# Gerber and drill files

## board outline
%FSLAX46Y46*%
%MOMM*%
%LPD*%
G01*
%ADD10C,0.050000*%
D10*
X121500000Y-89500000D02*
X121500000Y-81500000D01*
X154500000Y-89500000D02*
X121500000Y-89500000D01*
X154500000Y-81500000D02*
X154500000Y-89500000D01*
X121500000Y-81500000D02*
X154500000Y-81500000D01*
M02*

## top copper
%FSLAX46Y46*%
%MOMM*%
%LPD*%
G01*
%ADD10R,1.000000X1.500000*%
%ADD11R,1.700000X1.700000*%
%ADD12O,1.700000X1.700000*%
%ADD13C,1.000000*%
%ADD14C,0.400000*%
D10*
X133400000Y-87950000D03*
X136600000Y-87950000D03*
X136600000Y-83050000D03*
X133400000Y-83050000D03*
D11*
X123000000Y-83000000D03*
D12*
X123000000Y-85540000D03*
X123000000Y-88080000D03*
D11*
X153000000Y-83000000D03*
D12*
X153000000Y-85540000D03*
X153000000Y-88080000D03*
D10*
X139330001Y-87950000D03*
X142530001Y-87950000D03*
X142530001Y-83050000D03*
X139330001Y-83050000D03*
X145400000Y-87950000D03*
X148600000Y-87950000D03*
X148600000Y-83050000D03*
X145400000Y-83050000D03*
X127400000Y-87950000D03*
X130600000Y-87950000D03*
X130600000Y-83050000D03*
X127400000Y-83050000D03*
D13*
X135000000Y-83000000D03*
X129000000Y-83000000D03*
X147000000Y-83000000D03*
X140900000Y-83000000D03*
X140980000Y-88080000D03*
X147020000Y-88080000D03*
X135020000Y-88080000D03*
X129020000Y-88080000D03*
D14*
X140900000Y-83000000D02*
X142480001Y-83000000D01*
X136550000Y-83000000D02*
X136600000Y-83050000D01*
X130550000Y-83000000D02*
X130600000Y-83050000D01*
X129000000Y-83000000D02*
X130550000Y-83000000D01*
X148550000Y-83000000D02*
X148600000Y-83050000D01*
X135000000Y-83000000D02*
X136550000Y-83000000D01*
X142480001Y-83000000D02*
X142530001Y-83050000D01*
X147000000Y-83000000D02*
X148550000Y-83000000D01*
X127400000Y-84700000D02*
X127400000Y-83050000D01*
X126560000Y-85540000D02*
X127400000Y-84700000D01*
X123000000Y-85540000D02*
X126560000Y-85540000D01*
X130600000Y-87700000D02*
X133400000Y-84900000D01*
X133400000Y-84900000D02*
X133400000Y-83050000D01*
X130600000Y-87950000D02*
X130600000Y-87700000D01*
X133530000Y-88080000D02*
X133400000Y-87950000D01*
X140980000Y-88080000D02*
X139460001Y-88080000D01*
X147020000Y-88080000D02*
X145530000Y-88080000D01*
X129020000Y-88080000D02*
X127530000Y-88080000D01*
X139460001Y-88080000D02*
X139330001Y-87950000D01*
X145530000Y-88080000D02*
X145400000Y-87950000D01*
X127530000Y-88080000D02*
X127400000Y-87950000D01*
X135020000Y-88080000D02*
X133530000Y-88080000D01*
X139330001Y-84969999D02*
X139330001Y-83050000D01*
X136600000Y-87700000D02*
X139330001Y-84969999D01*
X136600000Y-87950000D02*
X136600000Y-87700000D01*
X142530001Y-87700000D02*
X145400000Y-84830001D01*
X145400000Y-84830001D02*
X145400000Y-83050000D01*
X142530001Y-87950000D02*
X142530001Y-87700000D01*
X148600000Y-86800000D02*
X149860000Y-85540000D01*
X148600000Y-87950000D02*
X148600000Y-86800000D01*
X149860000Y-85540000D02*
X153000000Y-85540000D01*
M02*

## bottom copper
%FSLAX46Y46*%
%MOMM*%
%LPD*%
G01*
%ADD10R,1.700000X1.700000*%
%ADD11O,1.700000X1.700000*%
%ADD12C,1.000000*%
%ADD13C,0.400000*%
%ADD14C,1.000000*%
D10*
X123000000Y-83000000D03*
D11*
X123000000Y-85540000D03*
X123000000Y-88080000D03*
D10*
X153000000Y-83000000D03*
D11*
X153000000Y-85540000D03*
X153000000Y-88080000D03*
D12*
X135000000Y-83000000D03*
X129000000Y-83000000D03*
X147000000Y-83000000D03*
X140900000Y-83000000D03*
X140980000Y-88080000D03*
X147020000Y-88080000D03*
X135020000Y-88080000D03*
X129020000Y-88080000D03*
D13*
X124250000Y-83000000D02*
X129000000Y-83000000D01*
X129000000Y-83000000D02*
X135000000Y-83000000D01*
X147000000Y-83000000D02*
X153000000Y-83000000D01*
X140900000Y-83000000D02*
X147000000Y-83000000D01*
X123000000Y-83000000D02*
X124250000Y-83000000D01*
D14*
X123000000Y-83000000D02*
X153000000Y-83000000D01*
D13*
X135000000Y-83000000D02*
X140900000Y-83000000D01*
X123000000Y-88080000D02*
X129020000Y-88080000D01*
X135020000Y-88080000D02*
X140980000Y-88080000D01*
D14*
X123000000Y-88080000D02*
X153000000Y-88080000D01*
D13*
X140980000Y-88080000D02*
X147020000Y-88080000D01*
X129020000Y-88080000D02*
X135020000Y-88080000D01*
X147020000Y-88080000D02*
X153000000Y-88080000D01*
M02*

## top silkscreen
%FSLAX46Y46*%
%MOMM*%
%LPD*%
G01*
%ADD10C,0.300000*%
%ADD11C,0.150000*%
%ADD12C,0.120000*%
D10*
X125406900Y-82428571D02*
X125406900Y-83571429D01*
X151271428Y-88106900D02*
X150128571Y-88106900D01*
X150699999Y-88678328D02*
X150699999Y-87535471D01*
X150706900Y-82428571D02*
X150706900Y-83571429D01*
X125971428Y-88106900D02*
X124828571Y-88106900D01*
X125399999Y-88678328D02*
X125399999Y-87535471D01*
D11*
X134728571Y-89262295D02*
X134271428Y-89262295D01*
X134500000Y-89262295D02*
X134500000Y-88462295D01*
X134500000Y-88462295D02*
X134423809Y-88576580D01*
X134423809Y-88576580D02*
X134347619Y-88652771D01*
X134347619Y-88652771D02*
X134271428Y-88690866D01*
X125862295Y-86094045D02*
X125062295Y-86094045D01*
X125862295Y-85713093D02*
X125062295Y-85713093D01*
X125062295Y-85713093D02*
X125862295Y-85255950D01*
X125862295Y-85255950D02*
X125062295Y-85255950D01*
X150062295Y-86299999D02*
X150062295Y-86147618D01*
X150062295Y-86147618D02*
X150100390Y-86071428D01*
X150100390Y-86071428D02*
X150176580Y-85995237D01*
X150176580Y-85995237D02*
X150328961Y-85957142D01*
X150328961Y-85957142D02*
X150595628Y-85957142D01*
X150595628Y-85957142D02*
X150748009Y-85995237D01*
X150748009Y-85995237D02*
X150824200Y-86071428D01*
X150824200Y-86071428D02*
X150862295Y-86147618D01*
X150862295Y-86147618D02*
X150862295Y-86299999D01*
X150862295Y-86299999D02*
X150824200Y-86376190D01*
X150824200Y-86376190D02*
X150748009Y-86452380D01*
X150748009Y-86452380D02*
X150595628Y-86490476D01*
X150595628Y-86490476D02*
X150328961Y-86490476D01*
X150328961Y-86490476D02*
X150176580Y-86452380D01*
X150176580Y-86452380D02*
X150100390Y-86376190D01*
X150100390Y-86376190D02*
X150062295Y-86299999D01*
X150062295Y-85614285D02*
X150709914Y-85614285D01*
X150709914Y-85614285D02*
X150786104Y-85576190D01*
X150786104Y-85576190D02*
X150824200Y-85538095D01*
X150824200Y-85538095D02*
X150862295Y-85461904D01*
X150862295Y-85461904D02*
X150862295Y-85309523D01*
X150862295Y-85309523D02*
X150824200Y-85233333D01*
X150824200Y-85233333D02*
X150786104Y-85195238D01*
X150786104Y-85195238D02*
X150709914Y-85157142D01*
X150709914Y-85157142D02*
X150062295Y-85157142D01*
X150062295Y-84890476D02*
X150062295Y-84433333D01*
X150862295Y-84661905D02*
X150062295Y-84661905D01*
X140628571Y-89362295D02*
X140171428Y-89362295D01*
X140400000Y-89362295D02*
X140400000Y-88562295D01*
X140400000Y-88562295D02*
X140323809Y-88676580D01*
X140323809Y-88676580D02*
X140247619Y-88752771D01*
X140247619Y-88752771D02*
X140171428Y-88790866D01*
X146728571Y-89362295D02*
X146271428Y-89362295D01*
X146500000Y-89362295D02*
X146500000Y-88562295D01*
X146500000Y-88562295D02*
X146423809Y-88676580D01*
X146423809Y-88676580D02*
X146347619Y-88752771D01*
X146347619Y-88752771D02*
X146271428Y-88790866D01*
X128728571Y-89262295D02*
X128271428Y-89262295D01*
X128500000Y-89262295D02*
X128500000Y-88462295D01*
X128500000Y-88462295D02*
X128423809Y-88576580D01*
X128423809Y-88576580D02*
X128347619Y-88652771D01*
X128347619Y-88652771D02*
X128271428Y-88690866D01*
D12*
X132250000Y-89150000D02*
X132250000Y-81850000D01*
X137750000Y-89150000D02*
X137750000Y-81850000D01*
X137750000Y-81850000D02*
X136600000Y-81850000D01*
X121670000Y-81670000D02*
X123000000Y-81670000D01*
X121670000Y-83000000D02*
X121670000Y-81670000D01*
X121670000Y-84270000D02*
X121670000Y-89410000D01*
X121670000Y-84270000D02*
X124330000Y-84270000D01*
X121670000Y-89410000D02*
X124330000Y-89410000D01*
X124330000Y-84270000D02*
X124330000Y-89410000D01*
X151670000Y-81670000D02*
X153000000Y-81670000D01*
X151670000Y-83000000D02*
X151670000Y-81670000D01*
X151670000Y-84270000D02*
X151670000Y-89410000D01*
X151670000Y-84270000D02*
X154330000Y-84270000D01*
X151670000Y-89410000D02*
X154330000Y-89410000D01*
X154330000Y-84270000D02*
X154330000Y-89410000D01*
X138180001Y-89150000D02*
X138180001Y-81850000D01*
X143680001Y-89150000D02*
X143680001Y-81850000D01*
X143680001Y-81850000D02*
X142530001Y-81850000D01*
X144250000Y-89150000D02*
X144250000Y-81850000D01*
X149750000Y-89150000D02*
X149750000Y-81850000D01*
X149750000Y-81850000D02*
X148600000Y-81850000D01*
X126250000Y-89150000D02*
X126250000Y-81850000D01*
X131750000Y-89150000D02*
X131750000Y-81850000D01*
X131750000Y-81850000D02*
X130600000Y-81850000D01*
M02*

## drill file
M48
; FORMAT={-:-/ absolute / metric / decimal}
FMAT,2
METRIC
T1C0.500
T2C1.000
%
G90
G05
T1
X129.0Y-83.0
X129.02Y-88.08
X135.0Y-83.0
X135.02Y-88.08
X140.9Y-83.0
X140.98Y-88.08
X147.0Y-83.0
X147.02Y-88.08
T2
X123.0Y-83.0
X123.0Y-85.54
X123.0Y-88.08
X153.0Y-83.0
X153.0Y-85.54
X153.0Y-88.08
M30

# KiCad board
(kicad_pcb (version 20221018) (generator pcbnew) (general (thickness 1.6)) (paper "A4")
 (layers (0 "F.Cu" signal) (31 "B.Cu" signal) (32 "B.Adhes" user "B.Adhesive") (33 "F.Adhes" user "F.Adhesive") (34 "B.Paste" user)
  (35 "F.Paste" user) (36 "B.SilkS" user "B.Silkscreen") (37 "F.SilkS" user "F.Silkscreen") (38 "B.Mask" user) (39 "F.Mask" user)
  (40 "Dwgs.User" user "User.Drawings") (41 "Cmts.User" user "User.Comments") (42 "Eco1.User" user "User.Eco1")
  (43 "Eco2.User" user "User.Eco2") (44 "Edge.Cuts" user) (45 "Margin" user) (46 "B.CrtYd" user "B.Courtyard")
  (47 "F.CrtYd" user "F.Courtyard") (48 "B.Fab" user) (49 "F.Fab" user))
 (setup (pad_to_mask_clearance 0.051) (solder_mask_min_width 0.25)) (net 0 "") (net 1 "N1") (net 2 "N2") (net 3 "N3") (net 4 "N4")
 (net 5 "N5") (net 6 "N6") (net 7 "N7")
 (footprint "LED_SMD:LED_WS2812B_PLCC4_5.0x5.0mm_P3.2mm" (layer "F.Cu") (at 135 85.5 90)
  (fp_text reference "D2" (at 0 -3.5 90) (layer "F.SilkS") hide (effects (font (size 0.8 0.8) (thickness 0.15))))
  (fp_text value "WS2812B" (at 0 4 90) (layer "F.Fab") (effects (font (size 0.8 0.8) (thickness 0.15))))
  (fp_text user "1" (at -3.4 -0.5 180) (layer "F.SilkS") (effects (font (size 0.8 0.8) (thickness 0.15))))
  (fp_line (start -3.65 -2.75) (end 3.65 -2.75) (stroke (width 0.12) (type solid)) (layer "F.SilkS"))
  (fp_line (start -3.65 2.75) (end 3.65 2.75) (stroke (width 0.12) (type solid)) (layer "F.SilkS"))
  (fp_line (start 3.65 2.75) (end 3.65 1.6) (stroke (width 0.12) (type solid)) (layer "F.SilkS"))
  (pad "1" smd rect (at -2.45 -1.6 90) (size 1.5 1) (layers "F.Cu" "F.Paste" "F.Mask") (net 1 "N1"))
  (pad "2" smd rect (at -2.45 1.6 90) (size 1.5 1) (layers "F.Cu" "F.Paste" "F.Mask") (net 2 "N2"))
  (pad "3" smd rect (at 2.45 1.6 90) (size 1.5 1) (layers "F.Cu" "F.Paste" "F.Mask") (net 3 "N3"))
  (pad "4" smd rect (at 2.45 -1.6 90) (size 1.5 1) (layers "F.Cu" "F.Paste" "F.Mask") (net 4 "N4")))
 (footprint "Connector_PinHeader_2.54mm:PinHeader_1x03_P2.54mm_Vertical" (layer "F.Cu") (at 123 83)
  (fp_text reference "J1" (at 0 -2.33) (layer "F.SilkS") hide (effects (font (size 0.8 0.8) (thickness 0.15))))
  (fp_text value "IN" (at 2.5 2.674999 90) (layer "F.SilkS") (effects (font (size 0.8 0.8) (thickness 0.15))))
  (fp_line (start -1.33 -1.33) (end 0 -1.33) (stroke (width 0.12) (type solid)) (layer "F.SilkS"))
  (fp_line (start -1.33 0) (end -1.33 -1.33) (stroke (width 0.12) (type solid)) (layer "F.SilkS"))
  (fp_line (start -1.33 1.27) (end -1.33 6.41) (stroke (width 0.12) (type solid)) (layer "F.SilkS"))
  (fp_line (start -1.33 1.27) (end 1.33 1.27) (stroke (width 0.12) (type solid)) (layer "F.SilkS"))
  (fp_line (start -1.33 6.41) (end 1.33 6.41) (stroke (width 0.12) (type solid)) (layer "F.SilkS"))
  (fp_line (start 1.33 1.27) (end 1.33 6.41) (stroke (width 0.12) (type solid)) (layer "F.SilkS"))
  (pad "1" thru_hole rect (at 0 0) (size 1.7 1.7) (drill 1) (layers "*.Cu" "*.Mask") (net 3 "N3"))
  (pad "2" thru_hole oval (at 0 2.54) (size 1.7 1.7) (drill 1) (layers "*.Cu" "*.Mask") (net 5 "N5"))
  (pad "3" thru_hole oval (at 0 5.08) (size 1.7 1.7) (drill 1) (layers "*.Cu" "*.Mask") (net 1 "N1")))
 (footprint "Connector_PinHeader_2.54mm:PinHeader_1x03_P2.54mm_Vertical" (layer "F.Cu") (at 153 83)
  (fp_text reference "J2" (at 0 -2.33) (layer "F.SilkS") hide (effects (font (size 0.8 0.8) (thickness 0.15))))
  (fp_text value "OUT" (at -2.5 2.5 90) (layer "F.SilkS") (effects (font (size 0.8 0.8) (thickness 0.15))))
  (fp_line (start -1.33 -1.33) (end 0 -1.33) (stroke (width 0.12) (type solid)) (layer "F.SilkS"))
  (fp_line (start -1.33 0) (end -1.33 -1.33) (stroke (width 0.12) (type solid)) (layer "F.SilkS"))
  (fp_line (start -1.33 1.27) (end -1.33 6.41) (stroke (width 0.12) (type solid)) (layer "F.SilkS"))
  (fp_line (start -1.33 1.27) (end 1.33 1.27) (stroke (width 0.12) (type solid)) (layer "F.SilkS"))
  (fp_line (start -1.33 6.41) (end 1.33 6.41) (stroke (width 0.12) (type solid)) (layer "F.SilkS"))
  (fp_line (start 1.33 1.27) (end 1.33 6.41) (stroke (width 0.12) (type solid)) (layer "F.SilkS"))
  (pad "1" thru_hole rect (at 0 0) (size 1.7 1.7) (drill 1) (layers "*.Cu" "*.Mask") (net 3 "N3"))
  (pad "2" thru_hole oval (at 0 2.54) (size 1.7 1.7) (drill 1) (layers "*.Cu" "*.Mask") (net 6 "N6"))
  (pad "3" thru_hole oval (at 0 5.08) (size 1.7 1.7) (drill 1) (layers "*.Cu" "*.Mask") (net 1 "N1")))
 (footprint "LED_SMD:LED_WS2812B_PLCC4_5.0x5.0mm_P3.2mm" (layer "F.Cu") (at 140.930001 85.5 90)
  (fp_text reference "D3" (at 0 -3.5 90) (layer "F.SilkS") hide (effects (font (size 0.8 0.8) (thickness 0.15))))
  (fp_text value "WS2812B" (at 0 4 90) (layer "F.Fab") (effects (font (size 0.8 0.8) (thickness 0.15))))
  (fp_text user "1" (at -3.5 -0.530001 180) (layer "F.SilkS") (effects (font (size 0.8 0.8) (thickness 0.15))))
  (fp_line (start -3.65 -2.75) (end 3.65 -2.75) (stroke (width 0.12) (type solid)) (layer "F.SilkS"))
  (fp_line (start -3.65 2.75) (end 3.65 2.75) (stroke (width 0.12) (type solid)) (layer "F.SilkS"))
  (fp_line (start 3.65 2.75) (end 3.65 1.6) (stroke (width 0.12) (type solid)) (layer "F.SilkS"))
  (pad "1" smd rect (at -2.45 -1.6 90) (size 1.5 1) (layers "F.Cu" "F.Paste" "F.Mask") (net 1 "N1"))
  (pad "2" smd rect (at -2.45 1.6 90) (size 1.5 1) (layers "F.Cu" "F.Paste" "F.Mask") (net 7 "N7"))
  (pad "3" smd rect (at 2.45 1.6 90) (size 1.5 1) (layers "F.Cu" "F.Paste" "F.Mask") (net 3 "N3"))
  (pad "4" smd rect (at 2.45 -1.6 90) (size 1.5 1) (layers "F.Cu" "F.Paste" "F.Mask") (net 2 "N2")))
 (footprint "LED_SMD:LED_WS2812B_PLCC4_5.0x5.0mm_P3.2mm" (layer "F.Cu") (at 147 85.5 90)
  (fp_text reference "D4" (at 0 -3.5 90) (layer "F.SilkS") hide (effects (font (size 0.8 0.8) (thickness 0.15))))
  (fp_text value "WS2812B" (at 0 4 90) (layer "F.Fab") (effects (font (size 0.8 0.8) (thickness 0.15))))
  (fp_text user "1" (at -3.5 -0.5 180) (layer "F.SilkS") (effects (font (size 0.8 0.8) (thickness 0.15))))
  (fp_line (start -3.65 -2.75) (end 3.65 -2.75) (stroke (width 0.12) (type solid)) (layer "F.SilkS"))
  (fp_line (start -3.65 2.75) (end 3.65 2.75) (stroke (width 0.12) (type solid)) (layer "F.SilkS"))
  (fp_line (start 3.65 2.75) (end 3.65 1.6) (stroke (width 0.12) (type solid)) (layer "F.SilkS"))
  (pad "1" smd rect (at -2.45 -1.6 90) (size 1.5 1) (layers "F.Cu" "F.Paste" "F.Mask") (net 1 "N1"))
  (pad "2" smd rect (at -2.45 1.6 90) (size 1.5 1) (layers "F.Cu" "F.Paste" "F.Mask") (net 6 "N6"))
  (pad "3" smd rect (at 2.45 1.6 90) (size 1.5 1) (layers "F.Cu" "F.Paste" "F.Mask") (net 3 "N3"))
  (pad "4" smd rect (at 2.45 -1.6 90) (size 1.5 1) (layers "F.Cu" "F.Paste" "F.Mask") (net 7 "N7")))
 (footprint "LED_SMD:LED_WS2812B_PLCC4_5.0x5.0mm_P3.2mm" (layer "F.Cu") (at 129 85.5 90)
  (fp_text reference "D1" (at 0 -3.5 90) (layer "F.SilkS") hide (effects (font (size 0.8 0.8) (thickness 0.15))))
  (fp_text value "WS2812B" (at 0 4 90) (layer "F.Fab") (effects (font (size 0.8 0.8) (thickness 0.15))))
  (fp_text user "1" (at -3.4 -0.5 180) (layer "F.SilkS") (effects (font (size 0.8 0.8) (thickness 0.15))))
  (fp_line (start -3.65 -2.75) (end 3.65 -2.75) (stroke (width 0.12) (type solid)) (layer "F.SilkS"))
  (fp_line (start -3.65 2.75) (end 3.65 2.75) (stroke (width 0.12) (type solid)) (layer "F.SilkS"))
  (fp_line (start 3.65 2.75) (end 3.65 1.6) (stroke (width 0.12) (type solid)) (layer "F.SilkS"))
  (pad "1" smd rect (at -2.45 -1.6 90) (size 1.5 1) (layers "F.Cu" "F.Paste" "F.Mask") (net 1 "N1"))
  (pad "2" smd rect (at -2.45 1.6 90) (size 1.5 1) (layers "F.Cu" "F.Paste" "F.Mask") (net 4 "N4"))
  (pad "3" smd rect (at 2.45 1.6 90) (size 1.5 1) (layers "F.Cu" "F.Paste" "F.Mask") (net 3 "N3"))
  (pad "4" smd rect (at 2.45 -1.6 90) (size 1.5 1) (layers "F.Cu" "F.Paste" "F.Mask") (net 5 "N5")))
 (gr_line (start 121.5 89.5) (end 121.5 81.5) (stroke (width 0.05) (type solid)) (layer "Edge.Cuts"))
 (gr_line (start 154.5 89.5) (end 121.5 89.5) (stroke (width 0.05) (type solid)) (layer "Edge.Cuts"))
 (gr_line (start 154.5 81.5) (end 154.5 89.5) (stroke (width 0.05) (type solid)) (layer "Edge.Cuts"))
 (gr_line (start 121.5 81.5) (end 154.5 81.5) (stroke (width 0.05) (type solid)) (layer "Edge.Cuts"))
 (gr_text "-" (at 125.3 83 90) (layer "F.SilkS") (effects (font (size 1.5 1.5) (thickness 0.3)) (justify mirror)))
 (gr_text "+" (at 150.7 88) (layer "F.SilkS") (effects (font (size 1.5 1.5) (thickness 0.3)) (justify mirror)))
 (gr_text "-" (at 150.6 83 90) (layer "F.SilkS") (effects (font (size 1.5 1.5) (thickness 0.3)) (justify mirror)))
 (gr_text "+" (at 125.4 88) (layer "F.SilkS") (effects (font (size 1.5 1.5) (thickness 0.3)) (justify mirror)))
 (segment (start 140.9 83) (end 142.480001 83) (width 0.4) (layer "F.Cu") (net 3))
 (segment (start 136.55 83) (end 136.6 83.05) (width 0.4) (layer "F.Cu") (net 3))
 (segment (start 130.55 83) (end 130.6 83.05) (width 0.4) (layer "F.Cu") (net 3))
 (segment (start 129 83) (end 130.55 83) (width 0.4) (layer "F.Cu") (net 3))
 (segment (start 148.55 83) (end 148.6 83.05) (width 0.4) (layer "F.Cu") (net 3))
 (segment (start 135 83) (end 136.55 83) (width 0.4) (layer "F.Cu") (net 3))
 (segment (start 142.480001 83) (end 142.530001 83.05) (width 0.4) (layer "F.Cu") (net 3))
 (segment (start 147 83) (end 148.55 83) (width 0.4) (layer "F.Cu") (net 3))
 (via (at 135 83) (size 1) (drill 0.5) (layers "F.Cu" "B.Cu") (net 3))
 (via (at 129 83) (size 1) (drill 0.5) (layers "F.Cu" "B.Cu") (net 3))
 (via (at 147 83) (size 1) (drill 0.5) (layers "F.Cu" "B.Cu") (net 3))
 (via (at 140.9 83) (size 1) (drill 0.5) (layers "F.Cu" "B.Cu") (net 3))
 (segment (start 124.25 83) (end 129 83) (width 0.4) (layer "B.Cu") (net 3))
 (segment (start 129 83) (end 135 83) (width 0.4) (layer "B.Cu") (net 3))
 (segment (start 147 83) (end 153 83) (width 0.4) (layer "B.Cu") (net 3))
 (segment (start 140.9 83) (end 147 83) (width 0.4) (layer "B.Cu") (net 3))
 (segment (start 123 83) (end 124.25 83) (width 0.4) (layer "B.Cu") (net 3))
 (segment (start 123 83) (end 153 83) (width 1) (layer "B.Cu") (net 3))
 (segment (start 135 83) (end 140.9 83) (width 0.4) (layer "B.Cu") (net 3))
 (segment (start 127.4 84.7) (end 127.4 83.05) (width 0.4) (layer "F.Cu") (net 5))
 (segment (start 126.56 85.54) (end 127.4 84.7) (width 0.4) (layer "F.Cu") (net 5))
 (segment (start 123 85.54) (end 126.56 85.54) (width 0.4) (layer "F.Cu") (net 5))
 (segment (start 130.6 87.7) (end 133.4 84.9) (width 0.4) (layer "F.Cu") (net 4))
 (segment (start 133.4 84.9) (end 133.4 83.05) (width 0.4) (layer "F.Cu") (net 4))
 (segment (start 130.6 87.95) (end 130.6 87.7) (width 0.4) (layer "F.Cu") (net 4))
 (segment (start 133.53 88.08) (end 133.4 87.95) (width 0.4) (layer "F.Cu") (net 1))
 (segment (start 140.98 88.08) (end 139.460001 88.08) (width 0.4) (layer "F.Cu") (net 1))
 (segment (start 147.02 88.08) (end 145.53 88.08) (width 0.4) (layer "F.Cu") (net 1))
 (segment (start 129.02 88.08) (end 127.53 88.08) (width 0.4) (layer "F.Cu") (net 1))
 (segment (start 139.460001 88.08) (end 139.330001 87.95) (width 0.4) (layer "F.Cu") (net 1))
 (segment (start 145.53 88.08) (end 145.4 87.95) (width 0.4) (layer "F.Cu") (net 1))
 (segment (start 127.53 88.08) (end 127.4 87.95) (width 0.4) (layer "F.Cu") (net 1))
 (segment (start 135.02 88.08) (end 133.53 88.08) (width 0.4) (layer "F.Cu") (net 1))
 (via (at 140.98 88.08) (size 1) (drill 0.5) (layers "F.Cu" "B.Cu") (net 1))
 (via (at 147.02 88.08) (size 1) (drill 0.5) (layers "F.Cu" "B.Cu") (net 1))
 (via (at 135.02 88.08) (size 1) (drill 0.5) (layers "F.Cu" "B.Cu") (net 1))
 (via (at 129.02 88.08) (size 1) (drill 0.5) (layers "F.Cu" "B.Cu") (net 1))
 (segment (start 123 88.08) (end 129.02 88.08) (width 0.4) (layer "B.Cu") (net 1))
 (segment (start 135.02 88.08) (end 140.98 88.08) (width 0.4) (layer "B.Cu") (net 1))
 (segment (start 123 88.08) (end 153 88.08) (width 1) (layer "B.Cu") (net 1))
 (segment (start 140.98 88.08) (end 147.02 88.08) (width 0.4) (layer "B.Cu") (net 1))
 (segment (start 129.02 88.08) (end 135.02 88.08) (width 0.4) (layer "B.Cu") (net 1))
 (segment (start 147.02 88.08) (end 153 88.08) (width 0.4) (layer "B.Cu") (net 1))
 (segment (start 139.330001 84.969999) (end 139.330001 83.05) (width 0.4) (layer "F.Cu") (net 2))
 (segment (start 136.6 87.7) (end 139.330001 84.969999) (width 0.4) (layer "F.Cu") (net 2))
 (segment (start 136.6 87.95) (end 136.6 87.7) (width 0.4) (layer "F.Cu") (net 2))
 (segment (start 142.530001 87.7) (end 145.4 84.830001) (width 0.4) (layer "F.Cu") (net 7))
 (segment (start 145.4 84.830001) (end 145.4 83.05) (width 0.4) (layer "F.Cu") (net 7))
 (segment (start 142.530001 87.95) (end 142.530001 87.7) (width 0.4) (layer "F.Cu") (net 7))
 (segment (start 148.6 86.8) (end 149.86 85.54) (width 0.4) (layer "F.Cu") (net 6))
 (segment (start 148.6 87.95) (end 148.6 86.8) (width 0.4) (layer "F.Cu") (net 6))
 (segment (start 149.86 85.54) (end 153 85.54) (width 0.4) (layer "F.Cu") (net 6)))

